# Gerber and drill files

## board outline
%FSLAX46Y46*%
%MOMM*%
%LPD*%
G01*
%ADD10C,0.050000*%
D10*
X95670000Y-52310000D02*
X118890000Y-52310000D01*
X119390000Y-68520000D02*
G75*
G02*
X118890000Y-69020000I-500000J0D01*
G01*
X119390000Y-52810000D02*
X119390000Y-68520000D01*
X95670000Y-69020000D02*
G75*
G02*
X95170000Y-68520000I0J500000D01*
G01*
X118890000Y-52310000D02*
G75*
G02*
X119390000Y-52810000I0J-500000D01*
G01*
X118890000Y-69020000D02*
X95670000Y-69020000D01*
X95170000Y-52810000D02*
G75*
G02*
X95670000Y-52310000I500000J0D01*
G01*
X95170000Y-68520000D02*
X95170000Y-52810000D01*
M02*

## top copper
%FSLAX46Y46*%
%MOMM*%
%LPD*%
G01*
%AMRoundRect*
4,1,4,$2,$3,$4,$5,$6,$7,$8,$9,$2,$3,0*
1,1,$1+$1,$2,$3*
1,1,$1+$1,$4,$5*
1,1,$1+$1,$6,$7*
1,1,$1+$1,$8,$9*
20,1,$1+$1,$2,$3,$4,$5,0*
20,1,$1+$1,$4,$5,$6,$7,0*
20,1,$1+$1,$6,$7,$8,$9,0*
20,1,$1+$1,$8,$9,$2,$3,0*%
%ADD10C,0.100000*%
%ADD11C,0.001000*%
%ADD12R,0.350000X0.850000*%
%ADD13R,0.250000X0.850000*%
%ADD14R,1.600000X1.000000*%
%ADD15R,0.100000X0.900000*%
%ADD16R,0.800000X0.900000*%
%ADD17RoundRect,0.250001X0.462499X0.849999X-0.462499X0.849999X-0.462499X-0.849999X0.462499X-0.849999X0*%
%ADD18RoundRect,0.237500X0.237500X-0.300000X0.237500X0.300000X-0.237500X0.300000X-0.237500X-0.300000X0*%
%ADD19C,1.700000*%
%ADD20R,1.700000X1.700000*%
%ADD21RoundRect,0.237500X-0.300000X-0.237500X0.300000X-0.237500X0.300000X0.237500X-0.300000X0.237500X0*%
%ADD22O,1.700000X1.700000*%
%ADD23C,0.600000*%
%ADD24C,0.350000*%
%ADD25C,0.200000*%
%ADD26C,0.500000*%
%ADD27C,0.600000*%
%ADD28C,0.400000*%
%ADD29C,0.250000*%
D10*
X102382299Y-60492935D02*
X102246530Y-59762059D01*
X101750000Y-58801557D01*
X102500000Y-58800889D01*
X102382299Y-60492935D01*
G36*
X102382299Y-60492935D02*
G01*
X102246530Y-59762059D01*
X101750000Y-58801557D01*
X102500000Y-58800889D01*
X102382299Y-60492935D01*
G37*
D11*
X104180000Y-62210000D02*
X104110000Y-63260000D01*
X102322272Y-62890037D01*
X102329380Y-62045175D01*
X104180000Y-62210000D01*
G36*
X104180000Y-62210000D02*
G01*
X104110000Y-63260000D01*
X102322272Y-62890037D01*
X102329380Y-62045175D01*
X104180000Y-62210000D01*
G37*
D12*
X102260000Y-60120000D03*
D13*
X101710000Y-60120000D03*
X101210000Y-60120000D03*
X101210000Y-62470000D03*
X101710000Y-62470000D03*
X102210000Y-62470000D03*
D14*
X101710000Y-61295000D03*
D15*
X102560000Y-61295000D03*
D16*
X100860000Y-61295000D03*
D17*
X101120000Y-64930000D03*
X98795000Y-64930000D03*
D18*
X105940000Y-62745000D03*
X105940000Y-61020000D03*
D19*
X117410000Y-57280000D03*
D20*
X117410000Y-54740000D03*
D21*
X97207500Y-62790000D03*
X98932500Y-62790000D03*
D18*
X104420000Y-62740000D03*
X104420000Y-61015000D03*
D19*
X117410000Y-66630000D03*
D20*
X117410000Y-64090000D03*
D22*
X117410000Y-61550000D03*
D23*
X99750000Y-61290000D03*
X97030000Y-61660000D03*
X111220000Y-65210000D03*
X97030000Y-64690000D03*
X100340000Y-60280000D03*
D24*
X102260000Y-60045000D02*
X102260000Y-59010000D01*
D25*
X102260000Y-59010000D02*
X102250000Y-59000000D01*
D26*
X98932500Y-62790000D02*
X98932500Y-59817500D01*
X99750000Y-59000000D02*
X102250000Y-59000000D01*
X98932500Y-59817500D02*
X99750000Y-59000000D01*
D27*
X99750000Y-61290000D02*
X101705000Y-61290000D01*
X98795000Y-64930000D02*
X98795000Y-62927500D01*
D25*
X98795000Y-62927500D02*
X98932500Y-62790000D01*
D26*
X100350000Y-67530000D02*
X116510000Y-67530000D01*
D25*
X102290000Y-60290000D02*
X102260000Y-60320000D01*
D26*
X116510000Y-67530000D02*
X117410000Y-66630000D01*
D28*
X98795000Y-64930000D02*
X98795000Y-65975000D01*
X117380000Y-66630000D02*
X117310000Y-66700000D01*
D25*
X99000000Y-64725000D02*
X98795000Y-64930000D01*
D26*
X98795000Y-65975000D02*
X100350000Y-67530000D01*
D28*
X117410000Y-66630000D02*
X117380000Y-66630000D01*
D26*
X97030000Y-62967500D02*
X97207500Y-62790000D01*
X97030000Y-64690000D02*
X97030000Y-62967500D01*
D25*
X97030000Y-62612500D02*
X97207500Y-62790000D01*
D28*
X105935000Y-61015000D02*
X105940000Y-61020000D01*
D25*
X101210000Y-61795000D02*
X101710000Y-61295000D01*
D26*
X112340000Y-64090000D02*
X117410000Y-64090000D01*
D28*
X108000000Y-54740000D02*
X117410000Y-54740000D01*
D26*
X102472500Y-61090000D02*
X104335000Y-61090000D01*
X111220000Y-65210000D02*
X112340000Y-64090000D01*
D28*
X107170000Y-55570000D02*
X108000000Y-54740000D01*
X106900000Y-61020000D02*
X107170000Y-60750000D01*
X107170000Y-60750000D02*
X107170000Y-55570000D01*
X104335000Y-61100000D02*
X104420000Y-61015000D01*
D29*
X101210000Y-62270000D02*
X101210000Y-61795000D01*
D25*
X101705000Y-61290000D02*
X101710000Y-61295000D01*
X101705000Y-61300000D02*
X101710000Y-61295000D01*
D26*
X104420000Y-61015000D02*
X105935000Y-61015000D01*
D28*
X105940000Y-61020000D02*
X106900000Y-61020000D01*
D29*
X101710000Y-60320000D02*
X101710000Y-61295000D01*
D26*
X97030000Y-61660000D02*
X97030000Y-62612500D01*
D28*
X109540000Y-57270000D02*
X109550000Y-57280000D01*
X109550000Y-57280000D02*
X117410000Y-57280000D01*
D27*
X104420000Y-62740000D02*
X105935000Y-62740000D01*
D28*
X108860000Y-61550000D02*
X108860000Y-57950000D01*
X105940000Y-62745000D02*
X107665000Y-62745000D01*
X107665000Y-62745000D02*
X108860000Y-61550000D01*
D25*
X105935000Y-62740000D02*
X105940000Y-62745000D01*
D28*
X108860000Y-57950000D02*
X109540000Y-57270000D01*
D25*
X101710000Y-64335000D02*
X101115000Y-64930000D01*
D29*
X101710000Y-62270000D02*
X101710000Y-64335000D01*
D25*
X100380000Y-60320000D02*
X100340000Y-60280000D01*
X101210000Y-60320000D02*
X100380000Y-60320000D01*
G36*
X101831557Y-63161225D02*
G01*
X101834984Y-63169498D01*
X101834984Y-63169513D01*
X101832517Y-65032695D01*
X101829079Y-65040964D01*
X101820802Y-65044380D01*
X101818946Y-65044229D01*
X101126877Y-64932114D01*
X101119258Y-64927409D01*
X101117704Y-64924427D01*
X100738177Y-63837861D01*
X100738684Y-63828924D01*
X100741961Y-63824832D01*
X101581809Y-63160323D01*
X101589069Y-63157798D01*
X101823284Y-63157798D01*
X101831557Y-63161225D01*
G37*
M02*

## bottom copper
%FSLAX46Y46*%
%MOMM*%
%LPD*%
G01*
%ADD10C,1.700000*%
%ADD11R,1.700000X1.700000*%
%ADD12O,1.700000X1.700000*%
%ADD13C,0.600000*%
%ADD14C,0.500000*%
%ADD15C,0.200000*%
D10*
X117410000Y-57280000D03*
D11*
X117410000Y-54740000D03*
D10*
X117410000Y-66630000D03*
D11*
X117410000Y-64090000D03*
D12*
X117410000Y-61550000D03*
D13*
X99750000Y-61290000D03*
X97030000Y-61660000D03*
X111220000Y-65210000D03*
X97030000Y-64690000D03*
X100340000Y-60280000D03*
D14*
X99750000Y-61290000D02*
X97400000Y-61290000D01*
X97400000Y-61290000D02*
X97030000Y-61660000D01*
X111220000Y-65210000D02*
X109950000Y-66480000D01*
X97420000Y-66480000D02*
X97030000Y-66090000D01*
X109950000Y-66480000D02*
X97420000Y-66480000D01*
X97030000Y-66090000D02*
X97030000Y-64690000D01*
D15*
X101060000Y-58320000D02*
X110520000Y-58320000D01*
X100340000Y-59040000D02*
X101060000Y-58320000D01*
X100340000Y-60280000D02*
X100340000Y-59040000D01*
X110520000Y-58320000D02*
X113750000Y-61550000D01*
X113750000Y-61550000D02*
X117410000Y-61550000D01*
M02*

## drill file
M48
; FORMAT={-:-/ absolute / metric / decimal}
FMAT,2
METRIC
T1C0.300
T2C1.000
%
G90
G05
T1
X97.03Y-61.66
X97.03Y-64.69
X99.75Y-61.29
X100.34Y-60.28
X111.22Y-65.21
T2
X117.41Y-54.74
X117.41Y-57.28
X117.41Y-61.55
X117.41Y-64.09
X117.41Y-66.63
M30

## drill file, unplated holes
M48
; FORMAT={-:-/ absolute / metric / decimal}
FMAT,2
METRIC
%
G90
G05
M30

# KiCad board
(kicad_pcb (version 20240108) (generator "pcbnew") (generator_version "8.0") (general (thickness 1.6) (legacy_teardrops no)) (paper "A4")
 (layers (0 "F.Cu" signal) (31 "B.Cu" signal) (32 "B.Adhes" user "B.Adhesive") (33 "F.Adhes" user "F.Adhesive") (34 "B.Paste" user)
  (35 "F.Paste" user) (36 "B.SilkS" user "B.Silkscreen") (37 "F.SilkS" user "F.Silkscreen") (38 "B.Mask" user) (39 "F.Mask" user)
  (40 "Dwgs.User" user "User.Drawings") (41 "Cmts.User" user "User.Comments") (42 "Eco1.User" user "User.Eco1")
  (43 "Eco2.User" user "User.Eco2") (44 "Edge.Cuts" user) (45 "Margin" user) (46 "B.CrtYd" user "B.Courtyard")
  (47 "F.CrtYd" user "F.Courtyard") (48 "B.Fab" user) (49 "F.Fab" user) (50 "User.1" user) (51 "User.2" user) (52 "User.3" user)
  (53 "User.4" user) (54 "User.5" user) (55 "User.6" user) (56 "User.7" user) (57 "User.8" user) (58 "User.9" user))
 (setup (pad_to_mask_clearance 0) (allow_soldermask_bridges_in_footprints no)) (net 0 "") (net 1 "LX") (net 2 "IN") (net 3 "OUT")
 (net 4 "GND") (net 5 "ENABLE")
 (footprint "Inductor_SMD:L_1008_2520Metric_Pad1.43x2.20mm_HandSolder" (layer "F.Cu") (at 99.9575 64.93 180)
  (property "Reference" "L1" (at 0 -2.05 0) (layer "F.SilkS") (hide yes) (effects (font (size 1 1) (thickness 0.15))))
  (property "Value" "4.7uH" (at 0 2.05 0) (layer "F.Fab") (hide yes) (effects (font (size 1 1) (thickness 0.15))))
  (pad "1" smd roundrect (at -1.1625 0 180) (size 1.425 2.2) (layers "F.Cu" "F.Paste" "F.Mask") (roundrect_rratio 0.175439) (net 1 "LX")
   (teardrops (best_length_ratio 0.5) (max_length 1) (best_width_ratio 1) (max_width 2) (curve_points 0) (filter_ratio 0.9) (enabled yes)
    (allow_two_segments yes) (prefer_zone_connections yes)))
  (pad "2" smd roundrect (at 1.1625 0 180) (size 1.425 2.2) (layers "F.Cu" "F.Paste" "F.Mask") (roundrect_rratio 0.175439) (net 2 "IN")))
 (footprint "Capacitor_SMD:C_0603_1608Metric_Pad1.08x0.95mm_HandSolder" (layer "F.Cu") (at 105.94 61.8825 90)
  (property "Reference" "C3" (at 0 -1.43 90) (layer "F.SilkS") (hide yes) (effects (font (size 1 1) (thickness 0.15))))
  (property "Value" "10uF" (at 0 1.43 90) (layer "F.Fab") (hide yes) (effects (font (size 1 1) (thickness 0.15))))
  (pad "1" smd roundrect (at -0.8625 0 90) (size 1.075 0.95) (layers "F.Cu" "F.Paste" "F.Mask") (roundrect_rratio 0.25) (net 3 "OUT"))
  (pad "2" smd roundrect (at 0.8625 0 90) (size 1.075 0.95) (layers "F.Cu" "F.Paste" "F.Mask") (roundrect_rratio 0.25) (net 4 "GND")))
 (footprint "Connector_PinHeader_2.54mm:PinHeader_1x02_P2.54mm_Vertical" (layer "F.Cu") (at 117.41 57.28 180)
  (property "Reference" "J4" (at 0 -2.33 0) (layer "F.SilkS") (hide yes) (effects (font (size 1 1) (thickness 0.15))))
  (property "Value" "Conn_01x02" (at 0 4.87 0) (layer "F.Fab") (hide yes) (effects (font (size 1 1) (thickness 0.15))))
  (pad "1" thru_hole circle (at 0 0 180) (size 1.7 1.7) (drill 1) (layers "*.Cu" "*.Mask") (remove_unused_layers no) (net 3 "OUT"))
  (pad "2" thru_hole rect (at 0 2.54 180) (size 1.7 1.7) (drill 1) (layers "*.Cu" "*.Mask") (remove_unused_layers no) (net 4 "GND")))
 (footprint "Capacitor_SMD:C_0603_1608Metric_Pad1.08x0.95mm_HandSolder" (layer "F.Cu") (at 98.07 62.79)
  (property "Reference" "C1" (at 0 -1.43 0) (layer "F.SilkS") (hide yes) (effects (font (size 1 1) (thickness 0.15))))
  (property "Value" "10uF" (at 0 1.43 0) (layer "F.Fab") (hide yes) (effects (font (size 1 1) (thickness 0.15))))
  (pad "1" smd roundrect (at -0.8625 0) (size 1.075 0.95) (layers "F.Cu" "F.Paste" "F.Mask") (roundrect_rratio 0.25) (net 4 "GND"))
  (pad "2" smd roundrect (at 0.8625 0) (size 1.075 0.95) (layers "F.Cu" "F.Paste" "F.Mask") (roundrect_rratio 0.25) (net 2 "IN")))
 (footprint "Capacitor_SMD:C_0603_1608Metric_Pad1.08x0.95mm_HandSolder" (layer "F.Cu") (at 104.42 61.8775 90)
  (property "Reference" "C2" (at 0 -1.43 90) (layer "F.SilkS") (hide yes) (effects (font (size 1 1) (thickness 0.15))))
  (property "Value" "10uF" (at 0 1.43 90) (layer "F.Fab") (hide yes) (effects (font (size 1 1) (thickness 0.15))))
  (pad "1" smd roundrect (at -0.8625 0 90) (size 1.075 0.95) (layers "F.Cu" "F.Paste" "F.Mask") (roundrect_rratio 0.25) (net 3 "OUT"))
  (pad "2" smd roundrect (at 0.8625 0 90) (size 1.075 0.95) (layers "F.Cu" "F.Paste" "F.Mask") (roundrect_rratio 0.25) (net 4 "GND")))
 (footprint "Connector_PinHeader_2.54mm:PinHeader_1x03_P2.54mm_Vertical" (layer "F.Cu") (at 117.41 66.63 180)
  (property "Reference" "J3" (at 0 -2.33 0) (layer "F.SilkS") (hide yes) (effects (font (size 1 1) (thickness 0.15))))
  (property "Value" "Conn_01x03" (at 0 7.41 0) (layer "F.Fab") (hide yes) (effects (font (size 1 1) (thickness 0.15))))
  (pad "1" thru_hole circle (at 0 0 180) (size 1.7 1.7) (drill 1) (layers "*.Cu" "*.Mask") (remove_unused_layers no) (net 2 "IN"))
  (pad "2" thru_hole rect (at 0 2.54 180) (size 1.7 1.7) (drill 1) (layers "*.Cu" "*.Mask") (remove_unused_layers no) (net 4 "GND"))
  (pad "3" thru_hole oval (at 0 5.08 180) (size 1.7 1.7) (drill 1) (layers "*.Cu" "*.Mask") (remove_unused_layers no) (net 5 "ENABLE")))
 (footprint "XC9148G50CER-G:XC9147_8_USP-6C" (layer "F.Cu") (at 101.71 61.295 -90)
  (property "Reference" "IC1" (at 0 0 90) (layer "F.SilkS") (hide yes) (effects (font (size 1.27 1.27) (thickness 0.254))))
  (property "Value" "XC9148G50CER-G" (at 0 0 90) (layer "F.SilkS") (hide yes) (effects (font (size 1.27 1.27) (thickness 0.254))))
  (pad "1" smd rect (at -1.175 -0.55) (size 0.35 0.85) (layers "F.Cu" "F.Paste" "F.Mask") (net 2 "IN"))
  (pad "2" smd rect (at -1.175 0) (size 0.25 0.85) (layers "F.Cu" "F.Paste" "F.Mask") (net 4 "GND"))
  (pad "3" smd rect (at -1.175 0.5) (size 0.25 0.85) (layers "F.Cu" "F.Paste" "F.Mask") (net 5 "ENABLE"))
  (pad "4" smd rect (at 1.175 0.5) (size 0.25 0.85) (layers "F.Cu" "F.Paste" "F.Mask") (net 4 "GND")
   (teardrops (best_length_ratio 0.5) (max_length 1) (best_width_ratio 1) (max_width 2) (curve_points 0) (filter_ratio 0.9) (enabled yes)
    (allow_two_segments yes) (prefer_zone_connections yes)))
  (pad "5" smd rect (at 1.175 0) (size 0.25 0.85) (layers "F.Cu" "F.Paste" "F.Mask") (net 1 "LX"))
  (pad "6" smd rect (at 1.175 -0.5) (size 0.25 0.85) (layers "F.Cu" "F.Paste" "F.Mask") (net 3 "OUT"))
  (pad "7" smd rect (at 0 0 270) (size 1 1.6) (layers "F.Cu" "F.Paste" "F.Mask") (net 4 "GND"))
  (pad "8" smd rect (at 0 -0.85) (size 0.1 0.9) (layers "F.Cu" "F.Paste" "F.Mask") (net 4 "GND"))
  (pad "9" smd rect (at 0 0.85) (size 0.8 0.9) (layers "F.Cu" "F.Paste" "F.Mask") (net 4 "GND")))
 (gr_poly
  (pts (xy 102.382299 60.492935) (xy 102.5 58.800889) (xy 101.75 58.801557) (xy 102.24653 59.762059)) (stroke (width 0.1) (type solid))
  (fill solid) (layer "F.Cu") (net 2))
 (gr_poly
  (pts (xy 102.32938 62.045175) (xy 104.18 62.21) (xy 104.11 63.26) (xy 102.322272 62.890037)) (stroke (width 0.001) (type solid))
  (fill solid) (layer "F.Cu") (net 3))
 (gr_line (start 95.67 52.31) (end 118.89 52.31) (stroke (width 0.05) (type default)) (layer "Edge.Cuts"))
 (gr_arc (start 119.39 68.52) (mid 119.243553 68.873553) (end 118.89 69.02) (stroke (width 0.05) (type default)) (layer "Edge.Cuts"))
 (gr_line (start 119.39 52.81) (end 119.39 68.52) (stroke (width 0.05) (type default)) (layer "Edge.Cuts"))
 (gr_arc (start 95.67 69.02) (mid 95.316447 68.873553) (end 95.17 68.52) (stroke (width 0.05) (type default)) (layer "Edge.Cuts"))
 (gr_arc (start 118.89 52.31) (mid 119.243553 52.456447) (end 119.39 52.81) (stroke (width 0.05) (type default)) (layer "Edge.Cuts"))
 (gr_line (start 118.89 69.02) (end 95.67 69.02) (stroke (width 0.05) (type default)) (layer "Edge.Cuts"))
 (gr_arc (start 95.17 52.81) (mid 95.316447 52.456447) (end 95.67 52.31) (stroke (width 0.05) (type default)) (layer "Edge.Cuts"))
 (gr_line (start 95.17 68.52) (end 95.17 52.81) (stroke (width 0.05) (type default)) (layer "Edge.Cuts"))
 (segment (start 98.795 64.93) (end 98.795 62.9275) (width 0.6) (layer "F.Cu") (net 2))
 (segment (start 98.795 62.9275) (end 98.9325 62.79) (width 0.2) (layer "F.Cu") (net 2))
 (segment (start 100.35 67.53) (end 116.51 67.53) (width 0.5) (layer "F.Cu") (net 2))
 (segment (start 102.29 60.29) (end 102.26 60.32) (width 0.2) (layer "F.Cu") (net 2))
 (segment (start 102.26 59.01) (end 102.25 59) (width 0.2) (layer "F.Cu") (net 2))
 (segment (start 98.9325 62.79) (end 98.9325 59.8175) (width 0.5) (layer "F.Cu") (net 2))
 (segment (start 116.51 67.53) (end 117.41 66.63) (width 0.5) (layer "F.Cu") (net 2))
 (segment (start 102.26 60.045) (end 102.26 59.01) (width 0.35) (layer "F.Cu") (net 2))
 (segment (start 99.75 59) (end 102.25 59) (width 0.5) (layer "F.Cu") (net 2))
 (segment (start 98.795 64.93) (end 98.795 65.975) (width 0.4) (layer "F.Cu") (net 2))
 (segment (start 117.38 66.63) (end 117.31 66.7) (width 0.4) (layer "F.Cu") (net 2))
 (segment (start 99 64.725) (end 98.795 64.93) (width 0.2) (layer "F.Cu") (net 2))
 (segment (start 98.795 65.975) (end 100.35 67.53) (width 0.5) (layer "F.Cu") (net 2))
 (segment (start 117.41 66.63) (end 117.38 66.63) (width 0.4) (layer "F.Cu") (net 2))
 (segment (start 98.9325 59.8175) (end 99.75 59) (width 0.5) (layer "F.Cu") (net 2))
 (segment (start 99.75 61.29) (end 101.705 61.29) (width 0.6) (layer "F.Cu") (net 4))
 (segment (start 97.03 62.9675) (end 97.2075 62.79) (width 0.5) (layer "F.Cu") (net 4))
 (segment (start 97.03 64.69) (end 97.03 62.9675) (width 0.5) (layer "F.Cu") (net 4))
 (segment (start 97.03 62.6125) (end 97.2075 62.79) (width 0.2) (layer "F.Cu") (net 4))
 (segment (start 105.935 61.015) (end 105.94 61.02) (width 0.4) (layer "F.Cu") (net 4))
 (segment (start 101.21 61.795) (end 101.71 61.295) (width 0.2) (layer "F.Cu") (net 4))
 (segment (start 112.34 64.09) (end 117.41 64.09) (width 0.5) (layer "F.Cu") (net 4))
 (segment (start 108 54.74) (end 117.41 54.74) (width 0.4) (layer "F.Cu") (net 4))
 (segment (start 102.4725 61.09) (end 104.335 61.09) (width 0.5) (layer "F.Cu") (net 4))
 (segment (start 111.22 65.21) (end 112.34 64.09) (width 0.5) (layer "F.Cu") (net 4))
 (segment (start 107.17 55.57) (end 108 54.74) (width 0.4) (layer "F.Cu") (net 4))
 (segment (start 106.9 61.02) (end 107.17 60.75) (width 0.4) (layer "F.Cu") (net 4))
 (segment (start 107.17 60.75) (end 107.17 55.57) (width 0.4) (layer "F.Cu") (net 4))
 (segment (start 104.335 61.1) (end 104.42 61.015) (width 0.4) (layer "F.Cu") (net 4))
 (segment (start 101.21 62.27) (end 101.21 61.795) (width 0.25) (layer "F.Cu") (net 4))
 (segment (start 101.705 61.29) (end 101.71 61.295) (width 0.2) (layer "F.Cu") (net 4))
 (segment (start 101.705 61.3) (end 101.71 61.295) (width 0.2) (layer "F.Cu") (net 4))
 (segment (start 104.42 61.015) (end 105.935 61.015) (width 0.5) (layer "F.Cu") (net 4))
 (segment (start 105.94 61.02) (end 106.9 61.02) (width 0.4) (layer "F.Cu") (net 4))
 (segment (start 101.71 60.32) (end 101.71 61.295) (width 0.25) (layer "F.Cu") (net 4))
 (segment (start 97.03 61.66) (end 97.03 62.6125) (width 0.5) (layer "F.Cu") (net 4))
 (via (at 99.75 61.29) (size 0.6) (drill 0.3) (layers "F.Cu" "B.Cu") (free yes) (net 4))
 (via (at 97.03 61.66) (size 0.6) (drill 0.3) (layers "F.Cu" "B.Cu") (free yes) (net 4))
 (via (at 111.22 65.21) (size 0.6) (drill 0.3) (layers "F.Cu" "B.Cu") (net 4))
 (via (at 97.03 64.69) (size 0.6) (drill 0.3) (layers "F.Cu" "B.Cu") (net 4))
 (segment (start 111.22 65.21) (end 109.95 66.48) (width 0.5) (layer "B.Cu") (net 4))
 (segment (start 99.75 61.29) (end 97.4 61.29) (width 0.5) (layer "B.Cu") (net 4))
 (segment (start 97.4 61.29) (end 97.03 61.66) (width 0.5) (layer "B.Cu") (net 4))
 (segment (start 97.42 66.48) (end 97.03 66.09) (width 0.5) (layer "B.Cu") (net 4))
 (segment (start 109.95 66.48) (end 97.42 66.48) (width 0.5) (layer "B.Cu") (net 4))
 (segment (start 97.03 66.09) (end 97.03 64.69) (width 0.5) (layer "B.Cu") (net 4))
 (segment (start 109.54 57.27) (end 109.55 57.28) (width 0.4) (layer "F.Cu") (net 3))
 (segment (start 109.55 57.28) (end 117.41 57.28) (width 0.4) (layer "F.Cu") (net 3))
 (segment (start 104.42 62.74) (end 105.935 62.74) (width 0.6) (layer "F.Cu") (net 3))
 (segment (start 108.86 61.55) (end 108.86 57.95) (width 0.4) (layer "F.Cu") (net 3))
 (segment (start 105.94 62.745) (end 107.665 62.745) (width 0.4) (layer "F.Cu") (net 3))
 (segment (start 107.665 62.745) (end 108.86 61.55) (width 0.4) (layer "F.Cu") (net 3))
 (segment (start 105.935 62.74) (end 105.94 62.745) (width 0.2) (layer "F.Cu") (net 3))
 (segment (start 108.86 57.95) (end 109.54 57.27) (width 0.4) (layer "F.Cu") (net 3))
 (segment (start 101.71 64.335) (end 101.115 64.93) (width 0.2) (layer "F.Cu") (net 1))
 (segment (start 101.71 62.27) (end 101.71 64.335) (width 0.25) (layer "F.Cu") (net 1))
 (segment (start 100.38 60.32) (end 100.34 60.28) (width 0.2) (layer "F.Cu") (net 5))
 (segment (start 101.21 60.32) (end 100.38 60.32) (width 0.2) (layer "F.Cu") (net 5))
 (via (at 100.34 60.28) (size 0.6) (drill 0.3) (layers "F.Cu" "B.Cu") (free yes) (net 5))
 (segment (start 101.06 58.32) (end 110.52 58.32) (width 0.2) (layer "B.Cu") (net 5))
 (segment (start 100.34 59.04) (end 101.06 58.32) (width 0.2) (layer "B.Cu") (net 5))
 (segment (start 100.34 60.28) (end 100.34 59.04) (width 0.2) (layer "B.Cu") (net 5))
 (segment (start 110.52 58.32) (end 113.75 61.55) (width 0.2) (layer "B.Cu") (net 5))
 (segment (start 113.75 61.55) (end 117.41 61.55) (width 0.2) (layer "B.Cu") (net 5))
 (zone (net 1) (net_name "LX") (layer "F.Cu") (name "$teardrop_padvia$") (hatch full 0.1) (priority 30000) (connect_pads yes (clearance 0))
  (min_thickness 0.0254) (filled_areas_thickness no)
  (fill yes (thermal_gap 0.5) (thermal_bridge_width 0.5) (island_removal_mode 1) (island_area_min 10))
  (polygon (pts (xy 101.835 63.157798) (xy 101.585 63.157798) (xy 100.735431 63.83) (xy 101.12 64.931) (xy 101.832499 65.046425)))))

